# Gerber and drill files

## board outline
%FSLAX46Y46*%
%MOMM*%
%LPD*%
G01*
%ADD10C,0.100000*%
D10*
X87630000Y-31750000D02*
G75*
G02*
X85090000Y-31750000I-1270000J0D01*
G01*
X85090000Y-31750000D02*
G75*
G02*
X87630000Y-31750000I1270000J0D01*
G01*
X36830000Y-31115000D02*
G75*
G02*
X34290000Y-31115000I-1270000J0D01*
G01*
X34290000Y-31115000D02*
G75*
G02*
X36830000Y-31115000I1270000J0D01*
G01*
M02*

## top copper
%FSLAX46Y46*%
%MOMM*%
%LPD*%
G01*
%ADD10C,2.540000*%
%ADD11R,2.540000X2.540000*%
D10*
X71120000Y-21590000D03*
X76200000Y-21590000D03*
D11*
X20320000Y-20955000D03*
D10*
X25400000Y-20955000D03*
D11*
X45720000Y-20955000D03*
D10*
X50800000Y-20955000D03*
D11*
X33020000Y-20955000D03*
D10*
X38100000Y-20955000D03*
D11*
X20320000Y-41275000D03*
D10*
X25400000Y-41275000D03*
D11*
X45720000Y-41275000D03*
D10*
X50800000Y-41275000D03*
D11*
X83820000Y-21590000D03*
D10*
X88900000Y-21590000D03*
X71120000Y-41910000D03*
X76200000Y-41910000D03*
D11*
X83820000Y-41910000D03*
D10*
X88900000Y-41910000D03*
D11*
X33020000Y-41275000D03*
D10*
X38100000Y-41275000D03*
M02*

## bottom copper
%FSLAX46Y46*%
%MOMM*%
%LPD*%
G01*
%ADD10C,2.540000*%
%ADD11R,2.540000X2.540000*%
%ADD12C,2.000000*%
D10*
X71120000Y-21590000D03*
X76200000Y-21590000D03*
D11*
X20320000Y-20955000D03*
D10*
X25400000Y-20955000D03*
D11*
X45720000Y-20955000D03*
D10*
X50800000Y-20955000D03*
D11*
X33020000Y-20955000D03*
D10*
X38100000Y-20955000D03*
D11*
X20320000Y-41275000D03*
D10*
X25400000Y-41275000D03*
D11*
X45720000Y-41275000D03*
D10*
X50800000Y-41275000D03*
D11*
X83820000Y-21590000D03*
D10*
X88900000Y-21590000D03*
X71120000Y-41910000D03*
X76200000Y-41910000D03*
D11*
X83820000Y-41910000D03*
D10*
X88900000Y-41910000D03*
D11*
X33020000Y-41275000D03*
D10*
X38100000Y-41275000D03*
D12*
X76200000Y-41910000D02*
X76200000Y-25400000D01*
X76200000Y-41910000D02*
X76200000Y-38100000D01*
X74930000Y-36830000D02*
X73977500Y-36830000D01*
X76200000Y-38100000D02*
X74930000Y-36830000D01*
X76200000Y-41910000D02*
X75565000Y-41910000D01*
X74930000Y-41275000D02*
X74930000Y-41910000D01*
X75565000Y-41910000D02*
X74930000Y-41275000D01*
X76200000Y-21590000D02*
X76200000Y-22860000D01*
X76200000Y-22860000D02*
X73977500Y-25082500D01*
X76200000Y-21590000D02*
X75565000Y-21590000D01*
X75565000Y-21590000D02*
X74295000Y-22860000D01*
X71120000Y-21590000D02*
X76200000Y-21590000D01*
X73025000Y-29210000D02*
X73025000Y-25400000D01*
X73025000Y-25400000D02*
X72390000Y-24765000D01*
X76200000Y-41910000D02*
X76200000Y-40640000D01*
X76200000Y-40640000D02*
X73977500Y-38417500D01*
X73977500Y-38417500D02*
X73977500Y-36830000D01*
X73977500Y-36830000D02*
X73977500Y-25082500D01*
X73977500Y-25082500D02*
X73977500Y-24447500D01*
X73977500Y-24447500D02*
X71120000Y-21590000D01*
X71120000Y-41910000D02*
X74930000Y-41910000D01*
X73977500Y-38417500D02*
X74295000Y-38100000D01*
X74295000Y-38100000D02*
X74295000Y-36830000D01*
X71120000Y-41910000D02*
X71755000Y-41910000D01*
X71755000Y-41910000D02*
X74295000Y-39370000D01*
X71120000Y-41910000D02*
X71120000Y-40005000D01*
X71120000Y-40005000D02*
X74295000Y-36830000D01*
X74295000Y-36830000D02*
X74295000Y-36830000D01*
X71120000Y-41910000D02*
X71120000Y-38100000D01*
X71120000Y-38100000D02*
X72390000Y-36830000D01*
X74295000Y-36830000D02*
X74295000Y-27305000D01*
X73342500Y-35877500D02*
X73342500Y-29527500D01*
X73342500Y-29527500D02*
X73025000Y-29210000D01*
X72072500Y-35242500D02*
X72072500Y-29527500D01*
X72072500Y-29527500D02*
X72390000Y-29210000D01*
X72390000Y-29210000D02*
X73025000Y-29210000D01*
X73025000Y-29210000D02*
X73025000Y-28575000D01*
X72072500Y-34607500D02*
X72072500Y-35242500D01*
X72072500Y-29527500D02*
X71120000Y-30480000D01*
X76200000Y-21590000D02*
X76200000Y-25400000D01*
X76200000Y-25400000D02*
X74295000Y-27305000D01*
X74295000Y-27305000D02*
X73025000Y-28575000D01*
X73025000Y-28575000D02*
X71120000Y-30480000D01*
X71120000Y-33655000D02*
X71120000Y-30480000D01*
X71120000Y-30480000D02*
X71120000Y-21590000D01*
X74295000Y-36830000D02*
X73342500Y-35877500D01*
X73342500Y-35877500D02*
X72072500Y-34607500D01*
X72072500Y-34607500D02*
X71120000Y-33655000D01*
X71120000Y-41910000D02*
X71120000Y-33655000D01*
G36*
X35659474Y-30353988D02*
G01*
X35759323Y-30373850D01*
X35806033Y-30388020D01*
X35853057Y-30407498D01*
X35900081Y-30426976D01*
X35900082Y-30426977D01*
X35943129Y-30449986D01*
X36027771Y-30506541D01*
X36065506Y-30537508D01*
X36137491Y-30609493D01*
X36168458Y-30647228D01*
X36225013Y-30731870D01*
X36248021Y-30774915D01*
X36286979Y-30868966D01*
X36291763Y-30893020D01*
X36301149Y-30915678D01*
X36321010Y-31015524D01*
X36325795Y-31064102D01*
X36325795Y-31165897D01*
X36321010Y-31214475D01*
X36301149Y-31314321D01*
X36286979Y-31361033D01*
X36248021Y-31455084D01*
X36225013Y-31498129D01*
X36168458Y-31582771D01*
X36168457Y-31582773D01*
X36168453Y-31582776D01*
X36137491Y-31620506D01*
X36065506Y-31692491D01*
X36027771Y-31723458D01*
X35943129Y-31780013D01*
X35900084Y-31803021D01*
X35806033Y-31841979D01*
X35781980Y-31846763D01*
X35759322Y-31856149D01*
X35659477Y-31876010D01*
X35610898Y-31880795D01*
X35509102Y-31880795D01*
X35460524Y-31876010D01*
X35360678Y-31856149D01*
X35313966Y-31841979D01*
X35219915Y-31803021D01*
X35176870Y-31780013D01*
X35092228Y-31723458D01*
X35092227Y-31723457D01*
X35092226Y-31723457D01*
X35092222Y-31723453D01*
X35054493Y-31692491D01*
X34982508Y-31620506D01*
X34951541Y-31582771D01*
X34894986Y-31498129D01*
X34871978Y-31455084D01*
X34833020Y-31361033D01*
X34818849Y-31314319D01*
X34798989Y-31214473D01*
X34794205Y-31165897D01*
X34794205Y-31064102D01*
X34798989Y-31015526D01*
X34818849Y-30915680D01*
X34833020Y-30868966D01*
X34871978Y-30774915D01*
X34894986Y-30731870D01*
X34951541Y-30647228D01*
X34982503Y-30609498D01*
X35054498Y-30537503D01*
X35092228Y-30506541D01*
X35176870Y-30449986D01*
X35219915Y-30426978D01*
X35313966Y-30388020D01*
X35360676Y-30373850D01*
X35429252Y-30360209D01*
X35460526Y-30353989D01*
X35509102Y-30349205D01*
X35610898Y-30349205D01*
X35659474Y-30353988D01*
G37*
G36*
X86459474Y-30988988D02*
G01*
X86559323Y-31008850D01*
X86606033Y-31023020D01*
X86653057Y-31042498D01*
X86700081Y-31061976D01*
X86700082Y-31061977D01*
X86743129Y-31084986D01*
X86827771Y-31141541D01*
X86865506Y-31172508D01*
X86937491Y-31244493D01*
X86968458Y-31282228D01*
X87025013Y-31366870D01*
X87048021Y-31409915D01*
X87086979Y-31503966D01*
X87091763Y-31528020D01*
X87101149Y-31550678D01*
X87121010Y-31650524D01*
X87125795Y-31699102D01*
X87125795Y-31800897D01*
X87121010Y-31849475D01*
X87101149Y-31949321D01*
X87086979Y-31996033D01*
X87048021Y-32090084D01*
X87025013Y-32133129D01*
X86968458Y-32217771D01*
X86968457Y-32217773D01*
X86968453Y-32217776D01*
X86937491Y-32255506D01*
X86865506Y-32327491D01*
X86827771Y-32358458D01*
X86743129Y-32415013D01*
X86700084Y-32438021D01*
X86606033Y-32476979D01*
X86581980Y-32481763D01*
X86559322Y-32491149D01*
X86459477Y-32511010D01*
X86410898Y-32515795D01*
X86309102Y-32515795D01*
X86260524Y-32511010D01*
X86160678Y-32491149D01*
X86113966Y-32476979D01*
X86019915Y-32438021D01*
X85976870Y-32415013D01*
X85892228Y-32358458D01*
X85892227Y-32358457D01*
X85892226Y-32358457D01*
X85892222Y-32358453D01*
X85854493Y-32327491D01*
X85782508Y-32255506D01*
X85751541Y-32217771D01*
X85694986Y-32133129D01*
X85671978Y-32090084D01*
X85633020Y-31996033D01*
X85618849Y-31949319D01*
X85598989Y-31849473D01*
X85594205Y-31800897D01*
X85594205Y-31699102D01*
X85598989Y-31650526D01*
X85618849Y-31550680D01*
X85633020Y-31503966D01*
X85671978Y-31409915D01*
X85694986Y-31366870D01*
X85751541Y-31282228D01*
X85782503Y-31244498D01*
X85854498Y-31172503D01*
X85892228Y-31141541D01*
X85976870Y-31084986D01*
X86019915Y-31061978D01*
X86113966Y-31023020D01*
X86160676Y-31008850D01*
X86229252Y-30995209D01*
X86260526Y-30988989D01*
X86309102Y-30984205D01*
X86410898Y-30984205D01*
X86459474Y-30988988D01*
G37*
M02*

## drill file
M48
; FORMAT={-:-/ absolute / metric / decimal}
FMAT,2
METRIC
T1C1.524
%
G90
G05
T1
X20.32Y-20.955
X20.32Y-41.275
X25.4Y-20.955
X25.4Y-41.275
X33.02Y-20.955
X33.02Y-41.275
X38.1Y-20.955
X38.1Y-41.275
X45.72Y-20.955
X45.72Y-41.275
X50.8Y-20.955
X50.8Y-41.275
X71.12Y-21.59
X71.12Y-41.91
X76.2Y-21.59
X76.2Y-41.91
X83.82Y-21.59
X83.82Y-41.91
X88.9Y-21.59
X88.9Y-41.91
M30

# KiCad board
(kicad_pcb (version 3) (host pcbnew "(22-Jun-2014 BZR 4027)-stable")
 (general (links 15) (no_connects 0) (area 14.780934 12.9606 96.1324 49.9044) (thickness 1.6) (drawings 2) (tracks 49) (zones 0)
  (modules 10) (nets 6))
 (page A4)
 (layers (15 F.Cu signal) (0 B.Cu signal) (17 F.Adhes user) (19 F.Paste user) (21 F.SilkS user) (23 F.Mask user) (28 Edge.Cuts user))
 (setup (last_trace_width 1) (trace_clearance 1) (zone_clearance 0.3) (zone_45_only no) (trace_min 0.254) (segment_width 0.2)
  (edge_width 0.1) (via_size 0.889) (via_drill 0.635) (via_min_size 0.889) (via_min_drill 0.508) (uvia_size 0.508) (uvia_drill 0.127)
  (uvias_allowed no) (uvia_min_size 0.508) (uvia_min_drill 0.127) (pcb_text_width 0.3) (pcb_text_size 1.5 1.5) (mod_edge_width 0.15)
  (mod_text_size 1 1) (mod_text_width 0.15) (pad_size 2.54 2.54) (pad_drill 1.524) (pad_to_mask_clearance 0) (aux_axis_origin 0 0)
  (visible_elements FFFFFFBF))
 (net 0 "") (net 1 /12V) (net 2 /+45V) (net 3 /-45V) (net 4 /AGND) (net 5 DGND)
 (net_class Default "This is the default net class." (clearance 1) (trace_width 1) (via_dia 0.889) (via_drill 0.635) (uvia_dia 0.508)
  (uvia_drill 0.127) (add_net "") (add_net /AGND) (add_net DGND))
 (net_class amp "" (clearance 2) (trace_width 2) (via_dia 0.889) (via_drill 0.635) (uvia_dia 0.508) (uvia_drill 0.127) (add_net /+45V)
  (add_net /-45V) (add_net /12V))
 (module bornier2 (layer F.Cu) (at 73.66 21.59)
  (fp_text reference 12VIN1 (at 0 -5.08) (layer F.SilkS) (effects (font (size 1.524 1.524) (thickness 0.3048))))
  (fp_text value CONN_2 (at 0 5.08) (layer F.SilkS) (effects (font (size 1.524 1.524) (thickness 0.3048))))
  (pad 1 thru_hole circle (at -2.54 0) (size 2.54 2.54) (drill 1.524) (layers *.Cu *.Mask F.SilkS) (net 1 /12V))
  (pad 2 thru_hole circle (at 2.54 0) (size 2.54 2.54) (drill 1.524) (layers *.Cu *.Mask F.SilkS) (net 1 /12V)))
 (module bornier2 (layer F.Cu) (at 22.86 20.955)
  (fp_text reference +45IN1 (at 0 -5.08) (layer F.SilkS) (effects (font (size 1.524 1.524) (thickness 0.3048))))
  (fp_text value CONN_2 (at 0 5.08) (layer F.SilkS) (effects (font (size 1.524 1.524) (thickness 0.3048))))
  (pad 1 thru_hole rect (at -2.54 0) (size 2.54 2.54) (drill 1.524) (layers *.Cu *.Mask F.SilkS) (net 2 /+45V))
  (pad 2 thru_hole circle (at 2.54 0) (size 2.54 2.54) (drill 1.524) (layers *.Cu *.Mask F.SilkS) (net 2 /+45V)))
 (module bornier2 (layer F.Cu) (at 48.26 20.955)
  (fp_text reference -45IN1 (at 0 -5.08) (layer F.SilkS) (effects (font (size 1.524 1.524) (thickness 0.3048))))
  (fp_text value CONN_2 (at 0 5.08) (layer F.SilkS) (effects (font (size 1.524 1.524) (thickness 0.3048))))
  (pad 1 thru_hole rect (at -2.54 0) (size 2.54 2.54) (drill 1.524) (layers *.Cu *.Mask F.SilkS) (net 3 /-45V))
  (pad 2 thru_hole circle (at 2.54 0) (size 2.54 2.54) (drill 1.524) (layers *.Cu *.Mask F.SilkS) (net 3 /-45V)))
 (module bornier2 (layer F.Cu) (at 35.56 20.955)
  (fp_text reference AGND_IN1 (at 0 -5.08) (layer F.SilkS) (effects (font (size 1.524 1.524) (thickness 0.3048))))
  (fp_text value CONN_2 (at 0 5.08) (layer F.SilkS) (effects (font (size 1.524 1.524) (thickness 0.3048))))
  (pad 1 thru_hole rect (at -2.54 0) (size 2.54 2.54) (drill 1.524) (layers *.Cu *.Mask F.SilkS) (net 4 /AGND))
  (pad 2 thru_hole circle (at 2.54 0) (size 2.54 2.54) (drill 1.524) (layers *.Cu *.Mask F.SilkS) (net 4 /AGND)))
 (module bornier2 (layer F.Cu) (at 22.86 41.275)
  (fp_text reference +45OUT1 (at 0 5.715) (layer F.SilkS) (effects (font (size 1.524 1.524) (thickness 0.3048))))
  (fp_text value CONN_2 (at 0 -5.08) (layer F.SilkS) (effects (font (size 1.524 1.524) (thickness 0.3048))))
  (pad 1 thru_hole rect (at -2.54 0) (size 2.54 2.54) (drill 1.524) (layers *.Cu *.Mask F.SilkS) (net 2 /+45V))
  (pad 2 thru_hole circle (at 2.54 0) (size 2.54 2.54) (drill 1.524) (layers *.Cu *.Mask F.SilkS) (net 2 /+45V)))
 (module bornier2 (layer F.Cu) (at 48.26 41.275)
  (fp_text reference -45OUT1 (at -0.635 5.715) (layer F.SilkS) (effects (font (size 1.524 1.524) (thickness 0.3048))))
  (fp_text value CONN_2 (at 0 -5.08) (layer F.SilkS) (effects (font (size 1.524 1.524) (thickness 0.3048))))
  (pad 1 thru_hole rect (at -2.54 0) (size 2.54 2.54) (drill 1.524) (layers *.Cu *.Mask F.SilkS) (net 3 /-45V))
  (pad 2 thru_hole circle (at 2.54 0) (size 2.54 2.54) (drill 1.524) (layers *.Cu *.Mask F.SilkS) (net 3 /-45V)))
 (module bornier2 (layer F.Cu) (at 86.36 21.59)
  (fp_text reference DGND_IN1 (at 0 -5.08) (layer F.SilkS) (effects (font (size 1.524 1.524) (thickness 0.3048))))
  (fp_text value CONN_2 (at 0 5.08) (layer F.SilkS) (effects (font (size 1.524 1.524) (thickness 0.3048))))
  (pad 1 thru_hole rect (at -2.54 0) (size 2.54 2.54) (drill 1.524) (layers *.Cu *.Mask F.SilkS) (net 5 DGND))
  (pad 2 thru_hole circle (at 2.54 0) (size 2.54 2.54) (drill 1.524) (layers *.Cu *.Mask F.SilkS) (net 5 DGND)))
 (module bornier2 (layer F.Cu) (at 73.66 41.91)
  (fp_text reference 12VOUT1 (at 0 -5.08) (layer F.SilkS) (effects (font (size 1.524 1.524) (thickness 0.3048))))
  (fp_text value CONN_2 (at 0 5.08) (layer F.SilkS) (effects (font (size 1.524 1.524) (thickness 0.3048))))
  (pad 1 thru_hole circle (at -2.54 0) (size 2.54 2.54) (drill 1.524) (layers *.Cu *.Mask F.SilkS) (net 1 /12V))
  (pad 2 thru_hole circle (at 2.54 0) (size 2.54 2.54) (drill 1.524) (layers *.Cu *.Mask F.SilkS) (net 1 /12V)))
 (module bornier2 (layer F.Cu) (at 86.36 41.91)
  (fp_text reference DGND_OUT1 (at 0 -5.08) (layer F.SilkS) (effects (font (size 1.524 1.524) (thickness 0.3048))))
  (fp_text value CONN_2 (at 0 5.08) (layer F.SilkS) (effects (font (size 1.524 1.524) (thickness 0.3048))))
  (pad 1 thru_hole rect (at -2.54 0) (size 2.54 2.54) (drill 1.524) (layers *.Cu *.Mask F.SilkS) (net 5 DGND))
  (pad 2 thru_hole circle (at 2.54 0) (size 2.54 2.54) (drill 1.524) (layers *.Cu *.Mask F.SilkS) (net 5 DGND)))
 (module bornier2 (layer F.Cu) (at 35.56 41.275)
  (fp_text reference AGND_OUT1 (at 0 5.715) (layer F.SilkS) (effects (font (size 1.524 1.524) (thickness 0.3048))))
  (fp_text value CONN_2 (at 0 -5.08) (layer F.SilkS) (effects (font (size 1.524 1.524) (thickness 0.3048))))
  (pad 1 thru_hole rect (at -2.54 0) (size 2.54 2.54) (drill 1.524) (layers *.Cu *.Mask F.SilkS) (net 4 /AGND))
  (pad 2 thru_hole circle (at 2.54 0) (size 2.54 2.54) (drill 1.524) (layers *.Cu *.Mask F.SilkS) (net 4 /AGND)))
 (gr_circle (center 86.36 31.75) (end 87.63 31.75) (layer Edge.Cuts) (width 0.1))
 (gr_circle (center 35.56 31.115) (end 36.83 31.115) (layer Edge.Cuts) (width 0.1))
 (segment (start 76.2 41.91) (end 76.2 25.4) (width 2) (layer B.Cu) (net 1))
 (segment (start 76.2 41.91) (end 76.2 38.1) (width 2) (layer B.Cu) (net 1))
 (segment (start 74.93 36.83) (end 73.9775 36.83) (width 2) (layer B.Cu) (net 1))
 (segment (start 76.2 38.1) (end 74.93 36.83) (width 2) (layer B.Cu) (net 1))
 (segment (start 76.2 41.91) (end 75.565 41.91) (width 2) (layer B.Cu) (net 1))
 (segment (start 74.93 41.275) (end 74.93 41.91) (width 2) (layer B.Cu) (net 1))
 (segment (start 75.565 41.91) (end 74.93 41.275) (width 2) (layer B.Cu) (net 1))
 (segment (start 76.2 21.59) (end 76.2 22.86) (width 2) (layer B.Cu) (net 1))
 (segment (start 76.2 22.86) (end 73.9775 25.0825) (width 2) (layer B.Cu) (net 1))
 (segment (start 76.2 21.59) (end 75.565 21.59) (width 2) (layer B.Cu) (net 1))
 (segment (start 75.565 21.59) (end 74.295 22.86) (width 2) (layer B.Cu) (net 1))
 (segment (start 71.12 21.59) (end 76.2 21.59) (width 2) (layer B.Cu) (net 1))
 (segment (start 73.025 29.21) (end 73.025 25.4) (width 2) (layer B.Cu) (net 1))
 (segment (start 73.025 25.4) (end 72.39 24.765) (width 2) (layer B.Cu) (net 1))
 (segment (start 76.2 41.91) (end 76.2 40.64) (width 2) (layer B.Cu) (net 1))
 (segment (start 76.2 40.64) (end 73.9775 38.4175) (width 2) (layer B.Cu) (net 1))
 (segment (start 73.9775 38.4175) (end 73.9775 36.83) (width 2) (layer B.Cu) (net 1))
 (segment (start 73.9775 36.83) (end 73.9775 25.0825) (width 2) (layer B.Cu) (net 1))
 (segment (start 73.9775 25.0825) (end 73.9775 24.4475) (width 2) (layer B.Cu) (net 1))
 (segment (start 73.9775 24.4475) (end 71.12 21.59) (width 2) (layer B.Cu) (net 1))
 (segment (start 71.12 41.91) (end 74.93 41.91) (width 2) (layer B.Cu) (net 1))
 (segment (start 73.9775 38.4175) (end 74.295 38.1) (width 2) (layer B.Cu) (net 1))
 (segment (start 74.295 38.1) (end 74.295 36.83) (width 2) (layer B.Cu) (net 1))
 (segment (start 71.12 41.91) (end 71.755 41.91) (width 2) (layer B.Cu) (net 1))
 (segment (start 71.755 41.91) (end 74.295 39.37) (width 2) (layer B.Cu) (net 1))
 (segment (start 71.12 41.91) (end 71.12 40.005) (width 2) (layer B.Cu) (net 1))
 (segment (start 71.12 40.005) (end 74.295 36.83) (width 2) (layer B.Cu) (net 1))
 (segment (start 74.295 36.83) (end 74.295 36.83) (width 2) (layer B.Cu) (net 1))
 (segment (start 71.12 41.91) (end 71.12 38.1) (width 2) (layer B.Cu) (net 1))
 (segment (start 71.12 38.1) (end 72.39 36.83) (width 2) (layer B.Cu) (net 1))
 (segment (start 74.295 36.83) (end 74.295 27.305) (width 2) (layer B.Cu) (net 1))
 (segment (start 73.3425 35.8775) (end 73.3425 29.5275) (width 2) (layer B.Cu) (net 1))
 (segment (start 73.3425 29.5275) (end 73.025 29.21) (width 2) (layer B.Cu) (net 1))
 (segment (start 72.0725 35.2425) (end 72.0725 29.5275) (width 2) (layer B.Cu) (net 1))
 (segment (start 72.0725 29.5275) (end 72.39 29.21) (width 2) (layer B.Cu) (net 1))
 (segment (start 72.39 29.21) (end 73.025 29.21) (width 2) (layer B.Cu) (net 1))
 (segment (start 73.025 29.21) (end 73.025 28.575) (width 2) (layer B.Cu) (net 1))
 (segment (start 72.0725 34.6075) (end 72.0725 35.2425) (width 2) (layer B.Cu) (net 1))
 (segment (start 72.0725 29.5275) (end 71.12 30.48) (width 2) (layer B.Cu) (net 1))
 (segment (start 76.2 21.59) (end 76.2 25.4) (width 2) (layer B.Cu) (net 1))
 (segment (start 76.2 25.4) (end 74.295 27.305) (width 2) (layer B.Cu) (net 1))
 (segment (start 74.295 27.305) (end 73.025 28.575) (width 2) (layer B.Cu) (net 1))
 (segment (start 73.025 28.575) (end 71.12 30.48) (width 2) (layer B.Cu) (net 1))
 (segment (start 71.12 33.655) (end 71.12 30.48) (width 2) (layer B.Cu) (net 1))
 (segment (start 71.12 30.48) (end 71.12 21.59) (width 2) (layer B.Cu) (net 1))
 (segment (start 74.295 36.83) (end 73.3425 35.8775) (width 2) (layer B.Cu) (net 1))
 (segment (start 73.3425 35.8775) (end 72.0725 34.6075) (width 2) (layer B.Cu) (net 1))
 (segment (start 72.0725 34.6075) (end 71.12 33.655) (width 2) (layer B.Cu) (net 1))
 (segment (start 71.12 41.91) (end 71.12 33.655) (width 2) (layer B.Cu) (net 1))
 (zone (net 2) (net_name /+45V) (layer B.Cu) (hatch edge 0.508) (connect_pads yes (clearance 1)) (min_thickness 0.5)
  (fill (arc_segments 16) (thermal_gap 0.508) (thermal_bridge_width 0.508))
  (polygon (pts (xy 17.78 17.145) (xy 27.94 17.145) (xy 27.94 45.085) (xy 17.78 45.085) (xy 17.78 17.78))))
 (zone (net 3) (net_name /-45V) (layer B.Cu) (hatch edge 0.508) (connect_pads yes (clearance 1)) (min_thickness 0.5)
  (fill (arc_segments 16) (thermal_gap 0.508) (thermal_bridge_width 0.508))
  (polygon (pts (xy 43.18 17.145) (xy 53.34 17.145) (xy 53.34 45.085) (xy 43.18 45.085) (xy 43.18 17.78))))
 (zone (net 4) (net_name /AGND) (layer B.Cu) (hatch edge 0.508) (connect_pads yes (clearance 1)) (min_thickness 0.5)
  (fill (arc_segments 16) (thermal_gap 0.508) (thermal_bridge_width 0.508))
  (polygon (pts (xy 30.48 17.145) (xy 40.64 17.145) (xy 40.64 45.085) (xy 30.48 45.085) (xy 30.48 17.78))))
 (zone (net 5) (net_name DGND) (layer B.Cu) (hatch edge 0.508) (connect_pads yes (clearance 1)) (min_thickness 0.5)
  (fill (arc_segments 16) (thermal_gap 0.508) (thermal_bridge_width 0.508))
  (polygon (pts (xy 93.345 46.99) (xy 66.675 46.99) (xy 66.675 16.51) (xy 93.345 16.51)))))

